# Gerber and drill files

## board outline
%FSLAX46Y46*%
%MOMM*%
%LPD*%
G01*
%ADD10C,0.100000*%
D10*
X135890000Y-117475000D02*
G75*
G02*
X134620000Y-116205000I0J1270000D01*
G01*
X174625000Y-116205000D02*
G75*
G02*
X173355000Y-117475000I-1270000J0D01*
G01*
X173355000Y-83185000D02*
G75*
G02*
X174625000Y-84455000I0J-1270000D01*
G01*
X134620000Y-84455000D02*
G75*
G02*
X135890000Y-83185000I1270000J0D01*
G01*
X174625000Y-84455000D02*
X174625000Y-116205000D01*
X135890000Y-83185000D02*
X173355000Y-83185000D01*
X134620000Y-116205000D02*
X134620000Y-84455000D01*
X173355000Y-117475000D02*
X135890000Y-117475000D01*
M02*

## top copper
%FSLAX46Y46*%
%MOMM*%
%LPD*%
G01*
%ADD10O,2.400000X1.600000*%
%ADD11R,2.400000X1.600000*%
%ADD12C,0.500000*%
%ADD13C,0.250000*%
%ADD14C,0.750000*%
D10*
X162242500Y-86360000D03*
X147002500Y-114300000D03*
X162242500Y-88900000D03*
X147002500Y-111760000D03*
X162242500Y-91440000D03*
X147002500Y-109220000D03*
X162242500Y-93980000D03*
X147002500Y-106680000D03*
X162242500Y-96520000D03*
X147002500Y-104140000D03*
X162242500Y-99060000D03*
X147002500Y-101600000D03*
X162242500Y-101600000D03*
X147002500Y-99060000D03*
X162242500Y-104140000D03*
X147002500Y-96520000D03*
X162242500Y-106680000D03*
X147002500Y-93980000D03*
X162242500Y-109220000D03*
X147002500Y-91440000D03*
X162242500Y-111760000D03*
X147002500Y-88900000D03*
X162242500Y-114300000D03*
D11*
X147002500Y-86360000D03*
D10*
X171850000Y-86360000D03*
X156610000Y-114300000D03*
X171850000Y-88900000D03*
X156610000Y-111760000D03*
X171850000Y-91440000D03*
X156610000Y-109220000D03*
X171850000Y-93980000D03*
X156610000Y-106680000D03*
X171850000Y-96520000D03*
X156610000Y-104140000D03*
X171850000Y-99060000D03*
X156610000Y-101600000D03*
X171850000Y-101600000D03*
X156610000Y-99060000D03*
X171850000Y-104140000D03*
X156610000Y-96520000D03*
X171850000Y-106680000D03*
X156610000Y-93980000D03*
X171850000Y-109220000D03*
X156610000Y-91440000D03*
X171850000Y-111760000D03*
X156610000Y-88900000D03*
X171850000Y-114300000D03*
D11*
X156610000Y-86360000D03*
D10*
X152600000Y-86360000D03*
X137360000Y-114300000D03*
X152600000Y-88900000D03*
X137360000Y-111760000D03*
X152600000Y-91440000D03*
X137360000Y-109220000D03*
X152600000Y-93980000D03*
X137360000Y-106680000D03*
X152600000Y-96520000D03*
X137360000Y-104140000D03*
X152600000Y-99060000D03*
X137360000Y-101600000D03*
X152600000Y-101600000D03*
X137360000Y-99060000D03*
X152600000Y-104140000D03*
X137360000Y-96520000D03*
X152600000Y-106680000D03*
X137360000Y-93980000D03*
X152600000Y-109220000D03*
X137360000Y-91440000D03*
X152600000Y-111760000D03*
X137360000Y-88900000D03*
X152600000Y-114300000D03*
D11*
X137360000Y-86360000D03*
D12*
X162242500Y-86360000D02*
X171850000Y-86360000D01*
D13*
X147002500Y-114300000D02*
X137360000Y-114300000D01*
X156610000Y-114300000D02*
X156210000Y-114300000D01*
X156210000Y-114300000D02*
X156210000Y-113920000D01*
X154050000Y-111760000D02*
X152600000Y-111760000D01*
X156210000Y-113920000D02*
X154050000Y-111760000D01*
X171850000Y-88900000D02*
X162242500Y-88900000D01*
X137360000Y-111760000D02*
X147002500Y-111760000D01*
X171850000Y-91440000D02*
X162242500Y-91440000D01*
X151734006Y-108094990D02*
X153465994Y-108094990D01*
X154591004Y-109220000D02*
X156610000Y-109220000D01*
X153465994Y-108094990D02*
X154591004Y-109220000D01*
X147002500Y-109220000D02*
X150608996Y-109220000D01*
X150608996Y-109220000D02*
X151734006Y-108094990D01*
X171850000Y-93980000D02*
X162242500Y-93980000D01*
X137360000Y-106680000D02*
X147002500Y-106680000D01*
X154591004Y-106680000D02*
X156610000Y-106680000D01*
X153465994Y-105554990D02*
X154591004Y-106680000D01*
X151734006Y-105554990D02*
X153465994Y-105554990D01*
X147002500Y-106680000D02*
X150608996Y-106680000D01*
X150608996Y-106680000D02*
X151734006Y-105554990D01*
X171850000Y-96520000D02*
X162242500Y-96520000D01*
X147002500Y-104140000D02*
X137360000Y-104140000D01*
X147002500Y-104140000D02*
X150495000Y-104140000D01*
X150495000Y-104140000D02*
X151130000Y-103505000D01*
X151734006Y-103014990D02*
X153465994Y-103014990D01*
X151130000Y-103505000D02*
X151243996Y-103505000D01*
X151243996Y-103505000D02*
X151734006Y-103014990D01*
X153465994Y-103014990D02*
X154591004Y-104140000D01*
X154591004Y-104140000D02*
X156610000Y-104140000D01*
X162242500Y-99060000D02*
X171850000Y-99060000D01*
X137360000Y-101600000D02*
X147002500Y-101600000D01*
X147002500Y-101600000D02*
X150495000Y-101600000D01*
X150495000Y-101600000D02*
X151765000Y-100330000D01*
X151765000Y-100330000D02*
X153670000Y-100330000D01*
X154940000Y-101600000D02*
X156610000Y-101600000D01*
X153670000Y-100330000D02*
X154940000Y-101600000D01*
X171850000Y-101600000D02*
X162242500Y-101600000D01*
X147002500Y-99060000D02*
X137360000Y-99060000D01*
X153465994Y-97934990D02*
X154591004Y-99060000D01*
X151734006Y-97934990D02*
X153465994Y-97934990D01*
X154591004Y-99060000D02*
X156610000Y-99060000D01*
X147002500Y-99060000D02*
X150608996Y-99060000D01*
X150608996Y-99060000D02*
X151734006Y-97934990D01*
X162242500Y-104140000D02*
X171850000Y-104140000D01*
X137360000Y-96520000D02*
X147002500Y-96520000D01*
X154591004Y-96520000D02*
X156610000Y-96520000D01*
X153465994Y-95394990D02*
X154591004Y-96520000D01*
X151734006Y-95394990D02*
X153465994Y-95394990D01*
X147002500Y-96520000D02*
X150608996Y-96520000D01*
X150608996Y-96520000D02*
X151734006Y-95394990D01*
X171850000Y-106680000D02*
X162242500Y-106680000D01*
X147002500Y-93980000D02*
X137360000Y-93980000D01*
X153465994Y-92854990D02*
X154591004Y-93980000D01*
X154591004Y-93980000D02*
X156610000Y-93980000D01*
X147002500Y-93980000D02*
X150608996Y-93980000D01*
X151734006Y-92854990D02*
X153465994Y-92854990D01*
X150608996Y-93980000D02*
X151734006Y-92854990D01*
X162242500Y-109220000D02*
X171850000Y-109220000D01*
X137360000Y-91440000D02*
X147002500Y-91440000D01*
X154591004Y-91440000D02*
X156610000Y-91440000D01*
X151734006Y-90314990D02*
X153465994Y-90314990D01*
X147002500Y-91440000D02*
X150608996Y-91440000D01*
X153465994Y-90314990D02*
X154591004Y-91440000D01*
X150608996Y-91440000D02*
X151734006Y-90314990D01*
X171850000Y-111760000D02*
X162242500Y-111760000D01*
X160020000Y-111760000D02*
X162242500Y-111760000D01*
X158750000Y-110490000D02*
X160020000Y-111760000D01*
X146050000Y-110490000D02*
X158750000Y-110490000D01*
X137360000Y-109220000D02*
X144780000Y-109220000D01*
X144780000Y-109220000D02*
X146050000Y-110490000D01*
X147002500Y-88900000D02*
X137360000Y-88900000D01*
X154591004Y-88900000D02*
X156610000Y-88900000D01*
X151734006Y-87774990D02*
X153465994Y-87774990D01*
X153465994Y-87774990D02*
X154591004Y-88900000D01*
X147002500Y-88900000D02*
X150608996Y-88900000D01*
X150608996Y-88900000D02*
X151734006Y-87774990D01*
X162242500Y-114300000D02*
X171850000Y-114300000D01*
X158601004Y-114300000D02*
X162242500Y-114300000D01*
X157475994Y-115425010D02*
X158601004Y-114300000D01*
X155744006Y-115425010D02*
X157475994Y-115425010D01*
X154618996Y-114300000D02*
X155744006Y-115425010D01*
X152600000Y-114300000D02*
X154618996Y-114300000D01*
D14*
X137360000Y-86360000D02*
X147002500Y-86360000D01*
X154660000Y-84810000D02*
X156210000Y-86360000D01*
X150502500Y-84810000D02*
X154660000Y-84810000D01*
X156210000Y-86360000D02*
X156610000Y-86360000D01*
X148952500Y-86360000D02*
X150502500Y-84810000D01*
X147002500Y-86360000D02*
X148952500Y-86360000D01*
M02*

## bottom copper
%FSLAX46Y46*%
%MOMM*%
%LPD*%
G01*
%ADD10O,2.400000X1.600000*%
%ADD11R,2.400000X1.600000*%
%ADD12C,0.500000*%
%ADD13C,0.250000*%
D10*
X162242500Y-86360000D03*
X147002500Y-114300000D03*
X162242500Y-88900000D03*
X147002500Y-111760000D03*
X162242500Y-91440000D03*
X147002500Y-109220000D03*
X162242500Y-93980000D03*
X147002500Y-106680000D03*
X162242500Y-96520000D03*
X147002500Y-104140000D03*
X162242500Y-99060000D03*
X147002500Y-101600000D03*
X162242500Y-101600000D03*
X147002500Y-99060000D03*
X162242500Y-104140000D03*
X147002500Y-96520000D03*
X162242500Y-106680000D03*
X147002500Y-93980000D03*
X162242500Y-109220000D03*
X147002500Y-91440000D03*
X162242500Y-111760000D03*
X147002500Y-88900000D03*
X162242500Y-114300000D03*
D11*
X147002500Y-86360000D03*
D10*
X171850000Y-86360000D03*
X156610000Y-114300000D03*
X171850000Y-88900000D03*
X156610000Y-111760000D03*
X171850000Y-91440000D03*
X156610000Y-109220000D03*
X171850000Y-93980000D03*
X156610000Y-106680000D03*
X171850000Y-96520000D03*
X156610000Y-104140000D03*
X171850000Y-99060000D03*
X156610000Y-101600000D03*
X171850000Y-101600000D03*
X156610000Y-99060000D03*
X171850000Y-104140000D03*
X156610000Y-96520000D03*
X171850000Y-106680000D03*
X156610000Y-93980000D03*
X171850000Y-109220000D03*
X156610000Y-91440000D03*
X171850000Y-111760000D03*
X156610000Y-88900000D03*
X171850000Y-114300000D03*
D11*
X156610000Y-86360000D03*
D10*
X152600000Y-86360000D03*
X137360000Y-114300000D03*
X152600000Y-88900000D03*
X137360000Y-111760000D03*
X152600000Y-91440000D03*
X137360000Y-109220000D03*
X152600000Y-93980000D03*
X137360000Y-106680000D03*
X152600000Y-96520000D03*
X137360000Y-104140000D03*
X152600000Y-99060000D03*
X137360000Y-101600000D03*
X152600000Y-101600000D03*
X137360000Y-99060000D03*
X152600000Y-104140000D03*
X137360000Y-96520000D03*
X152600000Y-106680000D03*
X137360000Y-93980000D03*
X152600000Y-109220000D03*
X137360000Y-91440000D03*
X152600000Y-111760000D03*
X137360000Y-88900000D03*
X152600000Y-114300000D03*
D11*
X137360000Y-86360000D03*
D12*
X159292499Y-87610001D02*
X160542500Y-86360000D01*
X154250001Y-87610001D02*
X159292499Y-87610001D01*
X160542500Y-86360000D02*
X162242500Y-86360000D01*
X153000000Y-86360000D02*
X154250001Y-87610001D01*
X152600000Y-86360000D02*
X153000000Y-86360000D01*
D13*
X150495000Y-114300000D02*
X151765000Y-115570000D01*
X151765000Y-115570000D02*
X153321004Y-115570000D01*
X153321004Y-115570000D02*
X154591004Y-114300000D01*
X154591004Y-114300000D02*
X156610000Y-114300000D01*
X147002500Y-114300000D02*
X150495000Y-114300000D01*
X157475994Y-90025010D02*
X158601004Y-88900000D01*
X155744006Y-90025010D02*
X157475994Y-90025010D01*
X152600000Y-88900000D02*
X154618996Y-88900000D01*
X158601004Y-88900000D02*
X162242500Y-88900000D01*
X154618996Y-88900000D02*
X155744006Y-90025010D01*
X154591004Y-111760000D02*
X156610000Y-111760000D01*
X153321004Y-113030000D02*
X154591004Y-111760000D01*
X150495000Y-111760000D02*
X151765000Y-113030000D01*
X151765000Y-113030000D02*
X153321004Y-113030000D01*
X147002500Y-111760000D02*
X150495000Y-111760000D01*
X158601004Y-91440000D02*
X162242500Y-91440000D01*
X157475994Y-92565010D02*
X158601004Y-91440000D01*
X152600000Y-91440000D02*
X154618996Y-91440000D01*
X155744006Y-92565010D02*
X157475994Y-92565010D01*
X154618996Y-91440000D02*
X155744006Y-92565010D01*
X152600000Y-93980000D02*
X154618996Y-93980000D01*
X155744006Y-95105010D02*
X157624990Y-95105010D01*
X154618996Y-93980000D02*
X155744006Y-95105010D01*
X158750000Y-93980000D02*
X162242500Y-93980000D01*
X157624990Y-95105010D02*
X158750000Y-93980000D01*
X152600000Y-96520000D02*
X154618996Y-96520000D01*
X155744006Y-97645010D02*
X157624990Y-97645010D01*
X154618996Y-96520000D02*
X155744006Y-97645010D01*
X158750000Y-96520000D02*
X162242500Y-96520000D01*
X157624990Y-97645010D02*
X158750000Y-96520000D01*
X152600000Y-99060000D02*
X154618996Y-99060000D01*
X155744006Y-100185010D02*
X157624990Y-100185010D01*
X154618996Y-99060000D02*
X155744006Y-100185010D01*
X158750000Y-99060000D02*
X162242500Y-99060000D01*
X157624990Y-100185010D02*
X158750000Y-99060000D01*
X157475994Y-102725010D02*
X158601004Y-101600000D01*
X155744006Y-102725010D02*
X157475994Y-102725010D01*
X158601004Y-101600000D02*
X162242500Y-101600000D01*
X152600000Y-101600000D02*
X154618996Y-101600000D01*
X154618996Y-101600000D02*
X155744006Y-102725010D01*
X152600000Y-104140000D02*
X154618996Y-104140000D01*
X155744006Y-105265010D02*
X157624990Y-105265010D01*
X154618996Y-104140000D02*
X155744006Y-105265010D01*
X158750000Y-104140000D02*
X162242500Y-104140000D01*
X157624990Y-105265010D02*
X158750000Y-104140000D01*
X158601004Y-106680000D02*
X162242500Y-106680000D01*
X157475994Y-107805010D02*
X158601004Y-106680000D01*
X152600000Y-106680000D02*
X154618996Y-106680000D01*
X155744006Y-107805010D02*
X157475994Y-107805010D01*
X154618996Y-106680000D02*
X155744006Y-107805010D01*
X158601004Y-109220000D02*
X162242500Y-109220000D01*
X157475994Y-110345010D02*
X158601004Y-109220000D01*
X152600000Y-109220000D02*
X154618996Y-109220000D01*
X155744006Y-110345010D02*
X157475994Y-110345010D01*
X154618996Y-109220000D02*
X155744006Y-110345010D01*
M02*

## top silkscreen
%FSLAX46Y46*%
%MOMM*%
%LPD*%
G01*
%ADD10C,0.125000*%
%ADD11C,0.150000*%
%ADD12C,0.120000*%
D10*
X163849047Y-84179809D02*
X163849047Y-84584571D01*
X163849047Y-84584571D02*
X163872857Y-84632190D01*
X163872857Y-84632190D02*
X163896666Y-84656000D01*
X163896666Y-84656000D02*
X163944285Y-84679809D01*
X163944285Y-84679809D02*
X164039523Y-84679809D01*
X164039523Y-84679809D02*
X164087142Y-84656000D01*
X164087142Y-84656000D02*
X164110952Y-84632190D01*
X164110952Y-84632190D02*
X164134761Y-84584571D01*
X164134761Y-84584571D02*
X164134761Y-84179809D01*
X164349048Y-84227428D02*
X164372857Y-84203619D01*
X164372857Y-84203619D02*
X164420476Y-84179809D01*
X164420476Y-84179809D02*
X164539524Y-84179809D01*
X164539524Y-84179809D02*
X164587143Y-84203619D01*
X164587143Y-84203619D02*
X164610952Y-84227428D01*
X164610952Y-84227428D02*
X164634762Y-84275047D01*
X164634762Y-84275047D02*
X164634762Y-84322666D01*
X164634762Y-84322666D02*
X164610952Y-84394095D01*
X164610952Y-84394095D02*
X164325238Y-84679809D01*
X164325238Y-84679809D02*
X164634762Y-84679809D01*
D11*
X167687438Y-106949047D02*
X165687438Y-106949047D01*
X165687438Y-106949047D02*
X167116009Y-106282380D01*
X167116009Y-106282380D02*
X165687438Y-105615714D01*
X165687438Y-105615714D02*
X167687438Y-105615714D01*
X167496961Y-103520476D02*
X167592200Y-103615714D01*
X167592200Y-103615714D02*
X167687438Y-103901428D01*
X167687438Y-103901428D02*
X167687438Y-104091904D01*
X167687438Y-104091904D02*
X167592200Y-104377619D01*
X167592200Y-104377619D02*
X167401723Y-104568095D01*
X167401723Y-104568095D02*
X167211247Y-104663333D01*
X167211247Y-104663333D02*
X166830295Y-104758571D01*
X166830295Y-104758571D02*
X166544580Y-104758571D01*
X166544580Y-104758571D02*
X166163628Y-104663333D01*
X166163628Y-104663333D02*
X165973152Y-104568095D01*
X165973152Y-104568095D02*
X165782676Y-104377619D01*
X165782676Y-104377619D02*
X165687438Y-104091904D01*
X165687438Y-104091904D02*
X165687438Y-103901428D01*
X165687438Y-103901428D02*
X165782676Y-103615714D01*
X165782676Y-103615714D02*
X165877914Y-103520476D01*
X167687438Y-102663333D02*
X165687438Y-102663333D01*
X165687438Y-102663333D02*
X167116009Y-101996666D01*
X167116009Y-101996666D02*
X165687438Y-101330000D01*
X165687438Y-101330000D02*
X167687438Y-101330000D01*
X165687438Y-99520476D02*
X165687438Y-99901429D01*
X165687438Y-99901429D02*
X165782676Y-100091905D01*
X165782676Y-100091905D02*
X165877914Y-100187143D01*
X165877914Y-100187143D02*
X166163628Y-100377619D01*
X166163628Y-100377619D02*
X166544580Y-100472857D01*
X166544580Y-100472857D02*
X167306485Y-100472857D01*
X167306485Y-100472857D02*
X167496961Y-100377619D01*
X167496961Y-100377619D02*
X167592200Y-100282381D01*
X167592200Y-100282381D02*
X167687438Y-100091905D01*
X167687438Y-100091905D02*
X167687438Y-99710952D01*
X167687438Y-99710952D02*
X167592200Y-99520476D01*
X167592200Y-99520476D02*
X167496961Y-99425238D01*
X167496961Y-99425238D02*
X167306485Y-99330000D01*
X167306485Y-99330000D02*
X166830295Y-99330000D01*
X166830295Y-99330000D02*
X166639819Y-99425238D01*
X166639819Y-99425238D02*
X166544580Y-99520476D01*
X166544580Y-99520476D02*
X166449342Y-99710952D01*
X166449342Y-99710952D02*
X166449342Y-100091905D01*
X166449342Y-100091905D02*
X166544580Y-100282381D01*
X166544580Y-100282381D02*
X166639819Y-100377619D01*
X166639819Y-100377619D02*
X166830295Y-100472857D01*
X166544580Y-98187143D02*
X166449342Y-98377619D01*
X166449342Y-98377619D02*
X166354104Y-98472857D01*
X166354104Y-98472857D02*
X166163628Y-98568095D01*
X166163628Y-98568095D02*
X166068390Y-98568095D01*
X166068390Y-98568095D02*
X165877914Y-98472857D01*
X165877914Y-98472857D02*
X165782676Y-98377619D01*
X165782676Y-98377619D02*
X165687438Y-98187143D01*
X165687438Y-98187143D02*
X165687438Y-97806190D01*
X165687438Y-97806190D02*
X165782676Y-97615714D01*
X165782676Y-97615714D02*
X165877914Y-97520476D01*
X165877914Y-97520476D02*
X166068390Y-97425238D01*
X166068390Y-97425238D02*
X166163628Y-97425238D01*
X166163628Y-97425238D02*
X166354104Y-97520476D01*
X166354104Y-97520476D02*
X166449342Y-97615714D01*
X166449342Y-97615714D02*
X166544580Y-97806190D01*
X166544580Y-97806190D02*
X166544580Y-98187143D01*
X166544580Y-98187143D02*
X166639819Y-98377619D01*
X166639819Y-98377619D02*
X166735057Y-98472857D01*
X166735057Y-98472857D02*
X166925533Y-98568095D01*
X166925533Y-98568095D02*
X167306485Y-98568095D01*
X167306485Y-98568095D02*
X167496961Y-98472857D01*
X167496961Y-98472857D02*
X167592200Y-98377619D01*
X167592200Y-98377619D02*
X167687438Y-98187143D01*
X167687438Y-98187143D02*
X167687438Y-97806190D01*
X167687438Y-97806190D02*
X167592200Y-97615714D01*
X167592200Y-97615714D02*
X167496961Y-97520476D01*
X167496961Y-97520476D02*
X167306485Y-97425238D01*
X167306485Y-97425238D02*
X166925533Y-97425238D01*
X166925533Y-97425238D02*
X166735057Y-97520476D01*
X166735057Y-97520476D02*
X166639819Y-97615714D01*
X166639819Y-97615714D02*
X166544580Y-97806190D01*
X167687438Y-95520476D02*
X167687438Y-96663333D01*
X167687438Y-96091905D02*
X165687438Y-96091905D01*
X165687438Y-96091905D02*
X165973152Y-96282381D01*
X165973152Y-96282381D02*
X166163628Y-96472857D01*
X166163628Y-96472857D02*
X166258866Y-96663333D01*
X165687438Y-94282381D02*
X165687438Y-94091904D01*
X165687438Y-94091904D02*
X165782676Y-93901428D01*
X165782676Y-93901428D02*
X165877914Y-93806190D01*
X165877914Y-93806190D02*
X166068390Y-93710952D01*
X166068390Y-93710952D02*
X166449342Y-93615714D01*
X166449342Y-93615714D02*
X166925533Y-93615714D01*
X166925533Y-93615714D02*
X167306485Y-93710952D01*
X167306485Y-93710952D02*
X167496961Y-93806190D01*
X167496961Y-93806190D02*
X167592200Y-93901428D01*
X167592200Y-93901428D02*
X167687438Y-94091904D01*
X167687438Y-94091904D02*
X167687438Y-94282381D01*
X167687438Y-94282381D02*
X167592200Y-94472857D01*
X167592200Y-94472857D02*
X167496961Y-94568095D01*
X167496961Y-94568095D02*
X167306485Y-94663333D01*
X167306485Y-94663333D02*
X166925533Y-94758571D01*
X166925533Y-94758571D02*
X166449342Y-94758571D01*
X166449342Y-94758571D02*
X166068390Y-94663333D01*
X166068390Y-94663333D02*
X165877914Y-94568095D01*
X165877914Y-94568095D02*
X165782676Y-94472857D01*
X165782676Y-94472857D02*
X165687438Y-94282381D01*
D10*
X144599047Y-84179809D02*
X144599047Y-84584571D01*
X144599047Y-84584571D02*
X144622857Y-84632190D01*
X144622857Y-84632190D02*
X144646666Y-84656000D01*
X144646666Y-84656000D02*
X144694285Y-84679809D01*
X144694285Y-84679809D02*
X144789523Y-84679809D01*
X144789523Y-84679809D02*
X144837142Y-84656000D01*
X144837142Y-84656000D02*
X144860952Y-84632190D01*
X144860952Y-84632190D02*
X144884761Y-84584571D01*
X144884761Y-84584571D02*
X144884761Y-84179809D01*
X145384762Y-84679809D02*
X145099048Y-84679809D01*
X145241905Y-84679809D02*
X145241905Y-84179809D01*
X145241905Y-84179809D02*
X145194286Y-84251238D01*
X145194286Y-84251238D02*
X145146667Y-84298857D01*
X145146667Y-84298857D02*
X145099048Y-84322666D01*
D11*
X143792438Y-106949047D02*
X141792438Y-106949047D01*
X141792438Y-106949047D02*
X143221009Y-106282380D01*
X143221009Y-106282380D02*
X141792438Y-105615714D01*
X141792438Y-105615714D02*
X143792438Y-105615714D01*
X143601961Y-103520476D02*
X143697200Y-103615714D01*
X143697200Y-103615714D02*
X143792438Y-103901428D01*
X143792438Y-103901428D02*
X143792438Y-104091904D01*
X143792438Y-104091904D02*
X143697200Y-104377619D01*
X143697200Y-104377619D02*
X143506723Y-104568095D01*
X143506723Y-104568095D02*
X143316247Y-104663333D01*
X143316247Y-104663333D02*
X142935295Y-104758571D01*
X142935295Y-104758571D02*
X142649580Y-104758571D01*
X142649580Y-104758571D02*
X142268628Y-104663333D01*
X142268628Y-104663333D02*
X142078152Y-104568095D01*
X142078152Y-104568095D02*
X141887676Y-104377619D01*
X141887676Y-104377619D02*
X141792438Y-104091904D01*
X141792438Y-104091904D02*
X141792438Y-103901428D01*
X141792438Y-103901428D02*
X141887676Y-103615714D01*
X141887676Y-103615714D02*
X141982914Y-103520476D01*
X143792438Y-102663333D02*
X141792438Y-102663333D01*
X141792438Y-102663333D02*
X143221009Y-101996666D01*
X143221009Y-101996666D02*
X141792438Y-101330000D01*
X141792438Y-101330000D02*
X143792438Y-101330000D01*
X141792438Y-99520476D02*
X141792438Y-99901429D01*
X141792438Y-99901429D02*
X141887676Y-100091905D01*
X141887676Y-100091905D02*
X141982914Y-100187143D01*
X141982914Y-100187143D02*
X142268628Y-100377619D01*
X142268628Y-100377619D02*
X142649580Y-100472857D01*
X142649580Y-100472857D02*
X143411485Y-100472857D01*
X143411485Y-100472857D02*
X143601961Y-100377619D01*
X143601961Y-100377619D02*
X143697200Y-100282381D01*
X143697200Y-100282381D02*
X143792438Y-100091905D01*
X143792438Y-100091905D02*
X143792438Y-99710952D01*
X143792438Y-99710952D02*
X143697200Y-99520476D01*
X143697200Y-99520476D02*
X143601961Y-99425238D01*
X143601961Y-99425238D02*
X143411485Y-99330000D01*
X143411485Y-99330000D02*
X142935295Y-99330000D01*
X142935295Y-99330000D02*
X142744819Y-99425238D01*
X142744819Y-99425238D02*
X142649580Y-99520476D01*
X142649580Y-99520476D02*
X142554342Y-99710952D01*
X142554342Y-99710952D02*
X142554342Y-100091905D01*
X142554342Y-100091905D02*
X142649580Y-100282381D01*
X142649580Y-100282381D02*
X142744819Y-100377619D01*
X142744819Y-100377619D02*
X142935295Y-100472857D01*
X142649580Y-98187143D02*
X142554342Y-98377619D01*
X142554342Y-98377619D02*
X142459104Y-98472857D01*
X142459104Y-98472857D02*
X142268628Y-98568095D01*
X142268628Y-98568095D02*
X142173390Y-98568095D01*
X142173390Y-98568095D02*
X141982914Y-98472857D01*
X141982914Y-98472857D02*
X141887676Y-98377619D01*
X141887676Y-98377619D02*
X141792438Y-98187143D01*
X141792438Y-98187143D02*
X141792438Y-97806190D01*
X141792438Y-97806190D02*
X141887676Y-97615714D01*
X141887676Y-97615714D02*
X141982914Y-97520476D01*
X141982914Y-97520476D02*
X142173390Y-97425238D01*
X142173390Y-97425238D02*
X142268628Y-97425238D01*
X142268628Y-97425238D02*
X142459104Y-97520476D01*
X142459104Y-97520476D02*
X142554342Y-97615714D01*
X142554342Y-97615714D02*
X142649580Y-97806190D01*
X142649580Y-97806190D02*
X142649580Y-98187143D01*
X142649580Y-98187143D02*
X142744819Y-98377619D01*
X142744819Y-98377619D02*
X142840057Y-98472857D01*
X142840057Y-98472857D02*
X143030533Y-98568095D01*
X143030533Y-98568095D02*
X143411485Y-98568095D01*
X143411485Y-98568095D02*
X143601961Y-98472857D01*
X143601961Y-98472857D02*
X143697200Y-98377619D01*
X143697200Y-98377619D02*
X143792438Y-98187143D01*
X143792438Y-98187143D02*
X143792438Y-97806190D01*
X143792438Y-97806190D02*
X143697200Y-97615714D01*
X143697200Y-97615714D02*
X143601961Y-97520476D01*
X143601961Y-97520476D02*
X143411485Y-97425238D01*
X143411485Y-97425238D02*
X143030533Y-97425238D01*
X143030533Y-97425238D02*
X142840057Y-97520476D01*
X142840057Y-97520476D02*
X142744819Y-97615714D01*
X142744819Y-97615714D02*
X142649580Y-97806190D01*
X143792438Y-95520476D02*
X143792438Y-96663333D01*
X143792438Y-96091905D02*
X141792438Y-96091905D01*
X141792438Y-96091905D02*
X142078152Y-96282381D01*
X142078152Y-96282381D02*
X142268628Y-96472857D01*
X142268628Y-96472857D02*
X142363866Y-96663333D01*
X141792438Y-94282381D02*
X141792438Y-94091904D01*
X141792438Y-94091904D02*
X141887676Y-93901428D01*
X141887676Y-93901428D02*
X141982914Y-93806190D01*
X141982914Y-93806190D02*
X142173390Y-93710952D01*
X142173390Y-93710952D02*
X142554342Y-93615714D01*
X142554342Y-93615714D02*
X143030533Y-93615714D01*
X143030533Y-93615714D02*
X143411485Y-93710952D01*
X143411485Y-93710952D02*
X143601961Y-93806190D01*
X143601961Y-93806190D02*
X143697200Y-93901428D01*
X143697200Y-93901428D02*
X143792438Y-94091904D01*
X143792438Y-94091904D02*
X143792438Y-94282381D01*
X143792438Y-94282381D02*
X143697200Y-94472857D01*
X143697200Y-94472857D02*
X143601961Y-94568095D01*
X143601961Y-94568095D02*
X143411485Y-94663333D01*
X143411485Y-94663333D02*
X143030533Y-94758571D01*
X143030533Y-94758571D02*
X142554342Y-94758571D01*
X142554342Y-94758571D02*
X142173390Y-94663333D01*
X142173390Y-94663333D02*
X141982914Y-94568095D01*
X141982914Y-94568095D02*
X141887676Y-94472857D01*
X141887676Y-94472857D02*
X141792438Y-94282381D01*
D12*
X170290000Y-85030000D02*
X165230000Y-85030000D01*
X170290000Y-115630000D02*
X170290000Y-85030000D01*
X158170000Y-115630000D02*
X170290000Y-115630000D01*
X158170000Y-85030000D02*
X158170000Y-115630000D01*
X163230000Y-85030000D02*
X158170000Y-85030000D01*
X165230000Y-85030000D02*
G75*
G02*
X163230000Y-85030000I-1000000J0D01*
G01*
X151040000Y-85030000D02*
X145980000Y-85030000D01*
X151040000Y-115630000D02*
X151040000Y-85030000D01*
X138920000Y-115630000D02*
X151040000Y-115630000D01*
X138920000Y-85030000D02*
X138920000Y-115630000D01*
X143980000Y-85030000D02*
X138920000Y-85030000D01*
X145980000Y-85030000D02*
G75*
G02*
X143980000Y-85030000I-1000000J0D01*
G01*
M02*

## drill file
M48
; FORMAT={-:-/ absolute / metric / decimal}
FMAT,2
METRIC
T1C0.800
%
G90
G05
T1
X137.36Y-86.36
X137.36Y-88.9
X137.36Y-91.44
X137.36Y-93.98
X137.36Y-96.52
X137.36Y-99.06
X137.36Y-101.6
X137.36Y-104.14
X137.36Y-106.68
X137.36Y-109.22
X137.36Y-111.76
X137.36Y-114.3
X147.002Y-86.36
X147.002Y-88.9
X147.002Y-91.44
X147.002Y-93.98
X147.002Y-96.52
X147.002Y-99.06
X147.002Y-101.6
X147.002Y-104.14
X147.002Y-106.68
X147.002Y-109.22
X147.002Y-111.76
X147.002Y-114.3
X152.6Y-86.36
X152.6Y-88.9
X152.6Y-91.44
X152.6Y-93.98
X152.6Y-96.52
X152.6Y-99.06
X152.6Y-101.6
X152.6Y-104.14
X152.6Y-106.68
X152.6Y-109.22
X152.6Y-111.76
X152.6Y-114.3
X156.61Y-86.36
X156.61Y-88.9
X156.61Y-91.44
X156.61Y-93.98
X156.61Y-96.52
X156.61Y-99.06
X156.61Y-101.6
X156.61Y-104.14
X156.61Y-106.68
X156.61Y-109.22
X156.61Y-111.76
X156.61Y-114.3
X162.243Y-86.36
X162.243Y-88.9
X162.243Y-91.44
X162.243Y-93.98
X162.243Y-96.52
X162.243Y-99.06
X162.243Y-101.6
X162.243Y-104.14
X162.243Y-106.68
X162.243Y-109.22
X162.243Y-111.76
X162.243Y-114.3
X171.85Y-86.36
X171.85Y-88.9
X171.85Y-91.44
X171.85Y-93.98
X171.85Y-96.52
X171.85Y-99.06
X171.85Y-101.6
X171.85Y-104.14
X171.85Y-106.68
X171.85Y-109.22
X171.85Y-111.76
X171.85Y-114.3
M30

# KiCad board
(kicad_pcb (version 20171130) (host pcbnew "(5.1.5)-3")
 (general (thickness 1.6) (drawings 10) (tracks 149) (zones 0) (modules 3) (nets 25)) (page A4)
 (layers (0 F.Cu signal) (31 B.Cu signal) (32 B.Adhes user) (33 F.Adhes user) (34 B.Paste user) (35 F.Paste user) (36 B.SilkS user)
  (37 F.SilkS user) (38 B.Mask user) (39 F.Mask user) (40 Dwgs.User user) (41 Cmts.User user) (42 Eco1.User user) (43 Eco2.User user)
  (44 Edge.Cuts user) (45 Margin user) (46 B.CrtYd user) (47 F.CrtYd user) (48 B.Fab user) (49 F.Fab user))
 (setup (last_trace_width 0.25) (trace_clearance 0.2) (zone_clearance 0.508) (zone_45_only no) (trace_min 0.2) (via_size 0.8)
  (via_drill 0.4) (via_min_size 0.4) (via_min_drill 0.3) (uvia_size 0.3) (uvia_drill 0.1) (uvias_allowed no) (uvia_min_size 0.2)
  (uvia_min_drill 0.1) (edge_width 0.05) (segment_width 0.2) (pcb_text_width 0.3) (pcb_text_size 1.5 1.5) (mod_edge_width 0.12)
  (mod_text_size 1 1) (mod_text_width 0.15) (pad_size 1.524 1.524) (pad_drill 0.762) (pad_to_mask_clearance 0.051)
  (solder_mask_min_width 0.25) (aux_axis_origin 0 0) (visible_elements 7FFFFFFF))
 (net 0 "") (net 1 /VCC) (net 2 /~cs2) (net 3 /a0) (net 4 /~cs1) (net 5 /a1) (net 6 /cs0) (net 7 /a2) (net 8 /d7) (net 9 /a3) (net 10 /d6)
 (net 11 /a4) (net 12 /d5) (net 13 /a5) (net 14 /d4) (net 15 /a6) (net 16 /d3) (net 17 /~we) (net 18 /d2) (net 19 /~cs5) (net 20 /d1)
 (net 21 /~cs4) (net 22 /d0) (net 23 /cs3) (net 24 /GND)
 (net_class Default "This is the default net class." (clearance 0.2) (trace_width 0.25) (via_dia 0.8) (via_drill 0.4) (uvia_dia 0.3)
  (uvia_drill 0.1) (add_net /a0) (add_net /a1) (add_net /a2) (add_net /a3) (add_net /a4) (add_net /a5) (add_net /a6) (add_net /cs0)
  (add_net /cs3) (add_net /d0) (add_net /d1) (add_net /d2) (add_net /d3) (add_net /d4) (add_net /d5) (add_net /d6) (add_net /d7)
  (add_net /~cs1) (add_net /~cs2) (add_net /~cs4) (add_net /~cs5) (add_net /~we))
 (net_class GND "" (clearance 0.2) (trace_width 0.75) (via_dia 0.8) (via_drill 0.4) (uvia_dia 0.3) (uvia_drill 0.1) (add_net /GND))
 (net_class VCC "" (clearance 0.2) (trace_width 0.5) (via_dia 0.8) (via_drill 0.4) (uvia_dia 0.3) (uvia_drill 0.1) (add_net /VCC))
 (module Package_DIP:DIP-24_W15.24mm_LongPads (layer F.Cu) (at 147.0025 86.36)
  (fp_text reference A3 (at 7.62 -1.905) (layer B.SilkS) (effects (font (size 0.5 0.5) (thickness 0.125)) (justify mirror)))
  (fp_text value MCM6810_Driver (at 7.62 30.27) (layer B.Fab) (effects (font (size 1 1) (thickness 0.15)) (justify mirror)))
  (pad 24 thru_hole oval (at 15.24 0) (size 2.4 1.6) (drill 0.8) (layers *.Cu *.Mask) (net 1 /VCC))
  (pad 12 thru_hole oval (at 0 27.94) (size 2.4 1.6) (drill 0.8) (layers *.Cu *.Mask) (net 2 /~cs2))
  (pad 23 thru_hole oval (at 15.24 2.54) (size 2.4 1.6) (drill 0.8) (layers *.Cu *.Mask) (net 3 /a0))
  (pad 11 thru_hole oval (at 0 25.4) (size 2.4 1.6) (drill 0.8) (layers *.Cu *.Mask) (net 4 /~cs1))
  (pad 22 thru_hole oval (at 15.24 5.08) (size 2.4 1.6) (drill 0.8) (layers *.Cu *.Mask) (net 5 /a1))
  (pad 10 thru_hole oval (at 0 22.86) (size 2.4 1.6) (drill 0.8) (layers *.Cu *.Mask) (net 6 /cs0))
  (pad 21 thru_hole oval (at 15.24 7.62) (size 2.4 1.6) (drill 0.8) (layers *.Cu *.Mask) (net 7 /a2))
  (pad 9 thru_hole oval (at 0 20.32) (size 2.4 1.6) (drill 0.8) (layers *.Cu *.Mask) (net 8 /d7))
  (pad 20 thru_hole oval (at 15.24 10.16) (size 2.4 1.6) (drill 0.8) (layers *.Cu *.Mask) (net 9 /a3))
  (pad 8 thru_hole oval (at 0 17.78) (size 2.4 1.6) (drill 0.8) (layers *.Cu *.Mask) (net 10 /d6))
  (pad 19 thru_hole oval (at 15.24 12.7) (size 2.4 1.6) (drill 0.8) (layers *.Cu *.Mask) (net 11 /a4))
  (pad 7 thru_hole oval (at 0 15.24) (size 2.4 1.6) (drill 0.8) (layers *.Cu *.Mask) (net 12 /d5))
  (pad 18 thru_hole oval (at 15.24 15.24) (size 2.4 1.6) (drill 0.8) (layers *.Cu *.Mask) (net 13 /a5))
  (pad 6 thru_hole oval (at 0 12.7) (size 2.4 1.6) (drill 0.8) (layers *.Cu *.Mask) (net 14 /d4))
  (pad 17 thru_hole oval (at 15.24 17.78) (size 2.4 1.6) (drill 0.8) (layers *.Cu *.Mask) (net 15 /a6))
  (pad 5 thru_hole oval (at 0 10.16) (size 2.4 1.6) (drill 0.8) (layers *.Cu *.Mask) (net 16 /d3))
  (pad 16 thru_hole oval (at 15.24 20.32) (size 2.4 1.6) (drill 0.8) (layers *.Cu *.Mask) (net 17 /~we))
  (pad 4 thru_hole oval (at 0 7.62) (size 2.4 1.6) (drill 0.8) (layers *.Cu *.Mask) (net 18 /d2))
  (pad 15 thru_hole oval (at 15.24 22.86) (size 2.4 1.6) (drill 0.8) (layers *.Cu *.Mask) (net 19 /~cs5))
  (pad 3 thru_hole oval (at 0 5.08) (size 2.4 1.6) (drill 0.8) (layers *.Cu *.Mask) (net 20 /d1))
  (pad 14 thru_hole oval (at 15.24 25.4) (size 2.4 1.6) (drill 0.8) (layers *.Cu *.Mask) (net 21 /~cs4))
  (pad 2 thru_hole oval (at 0 2.54) (size 2.4 1.6) (drill 0.8) (layers *.Cu *.Mask) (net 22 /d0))
  (pad 13 thru_hole oval (at 15.24 27.94) (size 2.4 1.6) (drill 0.8) (layers *.Cu *.Mask) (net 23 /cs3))
  (pad 1 thru_hole rect (at 0 0) (size 2.4 1.6) (drill 0.8) (layers *.Cu *.Mask) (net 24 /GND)))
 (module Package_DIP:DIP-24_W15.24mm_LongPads (layer F.Cu) (at 156.61 86.36)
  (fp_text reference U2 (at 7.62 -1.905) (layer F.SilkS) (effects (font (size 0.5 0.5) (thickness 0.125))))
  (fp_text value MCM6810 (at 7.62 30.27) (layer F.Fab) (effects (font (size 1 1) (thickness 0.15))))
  (fp_line (start 13.68 -1.33) (end 8.62 -1.33) (layer F.SilkS) (width 0.12))
  (fp_line (start 13.68 29.27) (end 13.68 -1.33) (layer F.SilkS) (width 0.12))
  (fp_line (start 1.56 29.27) (end 13.68 29.27) (layer F.SilkS) (width 0.12))
  (fp_line (start 1.56 -1.33) (end 1.56 29.27) (layer F.SilkS) (width 0.12))
  (fp_line (start 6.62 -1.33) (end 1.56 -1.33) (layer F.SilkS) (width 0.12))
  (fp_arc (start 7.62 -1.33) (end 6.62 -1.33) (angle -180) (layer F.SilkS) (width 0.12))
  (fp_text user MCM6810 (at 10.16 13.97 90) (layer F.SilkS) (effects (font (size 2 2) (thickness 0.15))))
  (pad 24 thru_hole oval (at 15.24 0) (size 2.4 1.6) (drill 0.8) (layers *.Cu *.Mask) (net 1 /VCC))
  (pad 12 thru_hole oval (at 0 27.94) (size 2.4 1.6) (drill 0.8) (layers *.Cu *.Mask) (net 2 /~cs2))
  (pad 23 thru_hole oval (at 15.24 2.54) (size 2.4 1.6) (drill 0.8) (layers *.Cu *.Mask) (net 3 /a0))
  (pad 11 thru_hole oval (at 0 25.4) (size 2.4 1.6) (drill 0.8) (layers *.Cu *.Mask) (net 4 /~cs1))
  (pad 22 thru_hole oval (at 15.24 5.08) (size 2.4 1.6) (drill 0.8) (layers *.Cu *.Mask) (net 5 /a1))
  (pad 10 thru_hole oval (at 0 22.86) (size 2.4 1.6) (drill 0.8) (layers *.Cu *.Mask) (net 6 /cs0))
  (pad 21 thru_hole oval (at 15.24 7.62) (size 2.4 1.6) (drill 0.8) (layers *.Cu *.Mask) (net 7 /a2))
  (pad 9 thru_hole oval (at 0 20.32) (size 2.4 1.6) (drill 0.8) (layers *.Cu *.Mask) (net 8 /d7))
  (pad 20 thru_hole oval (at 15.24 10.16) (size 2.4 1.6) (drill 0.8) (layers *.Cu *.Mask) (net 9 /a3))
  (pad 8 thru_hole oval (at 0 17.78) (size 2.4 1.6) (drill 0.8) (layers *.Cu *.Mask) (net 10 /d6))
  (pad 19 thru_hole oval (at 15.24 12.7) (size 2.4 1.6) (drill 0.8) (layers *.Cu *.Mask) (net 11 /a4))
  (pad 7 thru_hole oval (at 0 15.24) (size 2.4 1.6) (drill 0.8) (layers *.Cu *.Mask) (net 12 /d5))
  (pad 18 thru_hole oval (at 15.24 15.24) (size 2.4 1.6) (drill 0.8) (layers *.Cu *.Mask) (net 13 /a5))
  (pad 6 thru_hole oval (at 0 12.7) (size 2.4 1.6) (drill 0.8) (layers *.Cu *.Mask) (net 14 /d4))
  (pad 17 thru_hole oval (at 15.24 17.78) (size 2.4 1.6) (drill 0.8) (layers *.Cu *.Mask) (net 15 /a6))
  (pad 5 thru_hole oval (at 0 10.16) (size 2.4 1.6) (drill 0.8) (layers *.Cu *.Mask) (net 16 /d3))
  (pad 16 thru_hole oval (at 15.24 20.32) (size 2.4 1.6) (drill 0.8) (layers *.Cu *.Mask) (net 17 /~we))
  (pad 4 thru_hole oval (at 0 7.62) (size 2.4 1.6) (drill 0.8) (layers *.Cu *.Mask) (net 18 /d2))
  (pad 15 thru_hole oval (at 15.24 22.86) (size 2.4 1.6) (drill 0.8) (layers *.Cu *.Mask) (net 19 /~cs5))
  (pad 3 thru_hole oval (at 0 5.08) (size 2.4 1.6) (drill 0.8) (layers *.Cu *.Mask) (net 20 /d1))
  (pad 14 thru_hole oval (at 15.24 25.4) (size 2.4 1.6) (drill 0.8) (layers *.Cu *.Mask) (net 21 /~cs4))
  (pad 2 thru_hole oval (at 0 2.54) (size 2.4 1.6) (drill 0.8) (layers *.Cu *.Mask) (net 22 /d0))
  (pad 13 thru_hole oval (at 15.24 27.94) (size 2.4 1.6) (drill 0.8) (layers *.Cu *.Mask) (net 23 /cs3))
  (pad 1 thru_hole rect (at 0 0) (size 2.4 1.6) (drill 0.8) (layers *.Cu *.Mask) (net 24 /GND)))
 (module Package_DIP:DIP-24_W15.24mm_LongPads (layer F.Cu) (at 137.36 86.36)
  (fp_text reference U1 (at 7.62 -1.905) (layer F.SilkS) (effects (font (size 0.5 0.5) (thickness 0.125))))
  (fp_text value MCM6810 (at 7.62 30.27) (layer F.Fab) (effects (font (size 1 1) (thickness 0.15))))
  (fp_line (start 13.68 -1.33) (end 8.62 -1.33) (layer F.SilkS) (width 0.12))
  (fp_line (start 13.68 29.27) (end 13.68 -1.33) (layer F.SilkS) (width 0.12))
  (fp_line (start 1.56 29.27) (end 13.68 29.27) (layer F.SilkS) (width 0.12))
  (fp_line (start 1.56 -1.33) (end 1.56 29.27) (layer F.SilkS) (width 0.12))
  (fp_line (start 6.62 -1.33) (end 1.56 -1.33) (layer F.SilkS) (width 0.12))
  (fp_arc (start 7.62 -1.33) (end 6.62 -1.33) (angle -180) (layer F.SilkS) (width 0.12))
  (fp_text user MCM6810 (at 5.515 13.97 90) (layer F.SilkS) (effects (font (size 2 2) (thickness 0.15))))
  (pad 24 thru_hole oval (at 15.24 0) (size 2.4 1.6) (drill 0.8) (layers *.Cu *.Mask) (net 1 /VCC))
  (pad 12 thru_hole oval (at 0 27.94) (size 2.4 1.6) (drill 0.8) (layers *.Cu *.Mask) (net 2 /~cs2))
  (pad 23 thru_hole oval (at 15.24 2.54) (size 2.4 1.6) (drill 0.8) (layers *.Cu *.Mask) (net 3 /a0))
  (pad 11 thru_hole oval (at 0 25.4) (size 2.4 1.6) (drill 0.8) (layers *.Cu *.Mask) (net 4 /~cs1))
  (pad 22 thru_hole oval (at 15.24 5.08) (size 2.4 1.6) (drill 0.8) (layers *.Cu *.Mask) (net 5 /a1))
  (pad 10 thru_hole oval (at 0 22.86) (size 2.4 1.6) (drill 0.8) (layers *.Cu *.Mask) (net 21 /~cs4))
  (pad 21 thru_hole oval (at 15.24 7.62) (size 2.4 1.6) (drill 0.8) (layers *.Cu *.Mask) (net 7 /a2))
  (pad 9 thru_hole oval (at 0 20.32) (size 2.4 1.6) (drill 0.8) (layers *.Cu *.Mask) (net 8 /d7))
  (pad 20 thru_hole oval (at 15.24 10.16) (size 2.4 1.6) (drill 0.8) (layers *.Cu *.Mask) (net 9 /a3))
  (pad 8 thru_hole oval (at 0 17.78) (size 2.4 1.6) (drill 0.8) (layers *.Cu *.Mask) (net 10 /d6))
  (pad 19 thru_hole oval (at 15.24 12.7) (size 2.4 1.6) (drill 0.8) (layers *.Cu *.Mask) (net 11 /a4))
  (pad 7 thru_hole oval (at 0 15.24) (size 2.4 1.6) (drill 0.8) (layers *.Cu *.Mask) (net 12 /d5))
  (pad 18 thru_hole oval (at 15.24 15.24) (size 2.4 1.6) (drill 0.8) (layers *.Cu *.Mask) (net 13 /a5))
  (pad 6 thru_hole oval (at 0 12.7) (size 2.4 1.6) (drill 0.8) (layers *.Cu *.Mask) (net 14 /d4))
  (pad 17 thru_hole oval (at 15.24 17.78) (size 2.4 1.6) (drill 0.8) (layers *.Cu *.Mask) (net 15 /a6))
  (pad 5 thru_hole oval (at 0 10.16) (size 2.4 1.6) (drill 0.8) (layers *.Cu *.Mask) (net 16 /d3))
  (pad 16 thru_hole oval (at 15.24 20.32) (size 2.4 1.6) (drill 0.8) (layers *.Cu *.Mask) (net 17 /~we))
  (pad 4 thru_hole oval (at 0 7.62) (size 2.4 1.6) (drill 0.8) (layers *.Cu *.Mask) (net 18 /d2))
  (pad 15 thru_hole oval (at 15.24 22.86) (size 2.4 1.6) (drill 0.8) (layers *.Cu *.Mask) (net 19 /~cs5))
  (pad 3 thru_hole oval (at 0 5.08) (size 2.4 1.6) (drill 0.8) (layers *.Cu *.Mask) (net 20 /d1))
  (pad 14 thru_hole oval (at 15.24 25.4) (size 2.4 1.6) (drill 0.8) (layers *.Cu *.Mask) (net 2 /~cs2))
  (pad 2 thru_hole oval (at 0 2.54) (size 2.4 1.6) (drill 0.8) (layers *.Cu *.Mask) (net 22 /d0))
  (pad 13 thru_hole oval (at 15.24 27.94) (size 2.4 1.6) (drill 0.8) (layers *.Cu *.Mask) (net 23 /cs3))
  (pad 1 thru_hole rect (at 0 0) (size 2.4 1.6) (drill 0.8) (layers *.Cu *.Mask) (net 24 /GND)))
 (gr_arc (start 135.89 116.205) (end 134.62 116.205) (angle -90) (layer Edge.Cuts) (width 0.1))
 (gr_arc (start 173.355 116.205) (end 173.355 117.475) (angle -90) (layer Edge.Cuts) (width 0.1))
 (gr_arc (start 173.355 84.455) (end 174.625 84.455) (angle -90) (layer Edge.Cuts) (width 0.1))
 (gr_arc (start 135.89 84.455) (end 135.89 83.185) (angle -90) (layer Edge.Cuts) (width 0.1))
 (gr_line (start 174.625 84.455) (end 174.625 116.205) (layer Edge.Cuts) (width 0.1))
 (gr_line (start 135.89 83.185) (end 173.355 83.185) (layer Edge.Cuts) (width 0.1))
 (gr_line (start 134.62 116.205) (end 134.62 84.455) (layer Edge.Cuts) (width 0.1))
 (gr_line (start 173.355 117.475) (end 135.89 117.475) (layer Edge.Cuts) (width 0.1))
 (segment (start 159.292499 87.610001) (end 160.5425 86.36) (width 0.5) (layer B.Cu) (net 1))
 (segment (start 154.250001 87.610001) (end 159.292499 87.610001) (width 0.5) (layer B.Cu) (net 1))
 (segment (start 160.5425 86.36) (end 162.2425 86.36) (width 0.5) (layer B.Cu) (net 1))
 (segment (start 153 86.36) (end 154.250001 87.610001) (width 0.5) (layer B.Cu) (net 1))
 (segment (start 152.6 86.36) (end 153 86.36) (width 0.5) (layer B.Cu) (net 1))
 (segment (start 162.2425 86.36) (end 171.85 86.36) (width 0.5) (layer F.Cu) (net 1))
 (segment (start 147.0025 114.3) (end 137.36 114.3) (width 0.25) (layer F.Cu) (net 2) (status 30))
 (segment (start 156.61 114.3) (end 156.21 114.3) (width 0.25) (layer F.Cu) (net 2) (status 30))
 (segment (start 156.21 114.3) (end 156.21 113.92) (width 0.25) (layer F.Cu) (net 2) (status 30))
 (segment (start 150.495 114.3) (end 151.765 115.57) (width 0.25) (layer B.Cu) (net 2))
 (segment (start 151.765 115.57) (end 153.321004 115.57) (width 0.25) (layer B.Cu) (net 2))
 (segment (start 153.321004 115.57) (end 154.591004 114.3) (width 0.25) (layer B.Cu) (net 2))
 (segment (start 154.591004 114.3) (end 156.61 114.3) (width 0.25) (layer B.Cu) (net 2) (status 20))
 (segment (start 147.0025 114.3) (end 150.495 114.3) (width 0.25) (layer B.Cu) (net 2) (status 10))
 (segment (start 154.05 111.76) (end 152.6 111.76) (width 0.25) (layer F.Cu) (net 2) (status 20))
 (segment (start 156.21 113.92) (end 154.05 111.76) (width 0.25) (layer F.Cu) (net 2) (status 10))
 (segment (start 171.85 88.9) (end 162.2425 88.9) (width 0.25) (layer F.Cu) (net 3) (status 30))
 (segment (start 157.475994 90.02501) (end 158.601004 88.9) (width 0.25) (layer B.Cu) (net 3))
 (segment (start 155.744006 90.02501) (end 157.475994 90.02501) (width 0.25) (layer B.Cu) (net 3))
 (segment (start 152.6 88.9) (end 154.618996 88.9) (width 0.25) (layer B.Cu) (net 3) (status 10))
 (segment (start 158.601004 88.9) (end 162.2425 88.9) (width 0.25) (layer B.Cu) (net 3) (status 20))
 (segment (start 154.618996 88.9) (end 155.744006 90.02501) (width 0.25) (layer B.Cu) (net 3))
 (segment (start 137.36 111.76) (end 147.0025 111.76) (width 0.25) (layer F.Cu) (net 4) (status 30))
 (segment (start 154.591004 111.76) (end 156.61 111.76) (width 0.25) (layer B.Cu) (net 4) (status 20))
 (segment (start 153.321004 113.03) (end 154.591004 111.76) (width 0.25) (layer B.Cu) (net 4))
 (segment (start 150.495 111.76) (end 151.765 113.03) (width 0.25) (layer B.Cu) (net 4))
 (segment (start 151.765 113.03) (end 153.321004 113.03) (width 0.25) (layer B.Cu) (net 4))
 (segment (start 147.0025 111.76) (end 150.495 111.76) (width 0.25) (layer B.Cu) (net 4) (status 10))
 (segment (start 171.85 91.44) (end 162.2425 91.44) (width 0.25) (layer F.Cu) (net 5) (status 30))
 (segment (start 158.601004 91.44) (end 162.2425 91.44) (width 0.25) (layer B.Cu) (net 5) (status 20))
 (segment (start 157.475994 92.56501) (end 158.601004 91.44) (width 0.25) (layer B.Cu) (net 5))
 (segment (start 152.6 91.44) (end 154.618996 91.44) (width 0.25) (layer B.Cu) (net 5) (status 10))
 (segment (start 155.744006 92.56501) (end 157.475994 92.56501) (width 0.25) (layer B.Cu) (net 5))
 (segment (start 154.618996 91.44) (end 155.744006 92.56501) (width 0.25) (layer B.Cu) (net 5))
 (segment (start 151.734006 108.09499) (end 153.465994 108.09499) (width 0.25) (layer F.Cu) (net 6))
 (segment (start 154.591004 109.22) (end 156.61 109.22) (width 0.25) (layer F.Cu) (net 6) (status 20))
 (segment (start 153.465994 108.09499) (end 154.591004 109.22) (width 0.25) (layer F.Cu) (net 6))
 (segment (start 147.0025 109.22) (end 150.608996 109.22) (width 0.25) (layer F.Cu) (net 6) (status 10))
 (segment (start 150.608996 109.22) (end 151.734006 108.09499) (width 0.25) (layer F.Cu) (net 6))
 (segment (start 171.85 93.98) (end 162.2425 93.98) (width 0.25) (layer F.Cu) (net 7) (status 30))
 (segment (start 152.6 93.98) (end 154.618996 93.98) (width 0.25) (layer B.Cu) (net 7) (status 10))
 (segment (start 155.744006 95.10501) (end 157.62499 95.10501) (width 0.25) (layer B.Cu) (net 7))
 (segment (start 154.618996 93.98) (end 155.744006 95.10501) (width 0.25) (layer B.Cu) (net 7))
 (segment (start 158.75 93.98) (end 162.2425 93.98) (width 0.25) (layer B.Cu) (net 7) (status 20))
 (segment (start 157.62499 95.10501) (end 158.75 93.98) (width 0.25) (layer B.Cu) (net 7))
 (segment (start 137.36 106.68) (end 147.0025 106.68) (width 0.25) (layer F.Cu) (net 8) (status 30))
 (segment (start 154.591004 106.68) (end 156.61 106.68) (width 0.25) (layer F.Cu) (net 8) (status 20))
 (segment (start 153.465994 105.55499) (end 154.591004 106.68) (width 0.25) (layer F.Cu) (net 8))
 (segment (start 151.734006 105.55499) (end 153.465994 105.55499) (width 0.25) (layer F.Cu) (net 8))
 (segment (start 147.0025 106.68) (end 150.608996 106.68) (width 0.25) (layer F.Cu) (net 8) (status 10))
 (segment (start 150.608996 106.68) (end 151.734006 105.55499) (width 0.25) (layer F.Cu) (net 8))
 (segment (start 171.85 96.52) (end 162.2425 96.52) (width 0.25) (layer F.Cu) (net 9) (status 30))
 (segment (start 152.6 96.52) (end 154.618996 96.52) (width 0.25) (layer B.Cu) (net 9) (status 10))
 (segment (start 155.744006 97.64501) (end 157.62499 97.64501) (width 0.25) (layer B.Cu) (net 9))
 (segment (start 154.618996 96.52) (end 155.744006 97.64501) (width 0.25) (layer B.Cu) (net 9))
 (segment (start 158.75 96.52) (end 162.2425 96.52) (width 0.25) (layer B.Cu) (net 9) (status 20))
 (segment (start 157.62499 97.64501) (end 158.75 96.52) (width 0.25) (layer B.Cu) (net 9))
 (segment (start 147.0025 104.14) (end 137.36 104.14) (width 0.25) (layer F.Cu) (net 10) (status 30))
 (segment (start 147.0025 104.14) (end 150.495 104.14) (width 0.25) (layer F.Cu) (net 10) (status 10))
 (segment (start 150.495 104.14) (end 151.13 103.505) (width 0.25) (layer F.Cu) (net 10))
 (segment (start 151.734006 103.01499) (end 153.465994 103.01499) (width 0.25) (layer F.Cu) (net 10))
 (segment (start 151.13 103.505) (end 151.243996 103.505) (width 0.25) (layer F.Cu) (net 10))
 (segment (start 151.243996 103.505) (end 151.734006 103.01499) (width 0.25) (layer F.Cu) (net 10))
 (segment (start 153.465994 103.01499) (end 154.591004 104.14) (width 0.25) (layer F.Cu) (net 10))
 (segment (start 154.591004 104.14) (end 156.61 104.14) (width 0.25) (layer F.Cu) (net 10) (status 20))
 (segment (start 162.2425 99.06) (end 171.85 99.06) (width 0.25) (layer F.Cu) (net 11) (status 30))
 (segment (start 152.6 99.06) (end 154.618996 99.06) (width 0.25) (layer B.Cu) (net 11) (status 10))
 (segment (start 155.744006 100.18501) (end 157.62499 100.18501) (width 0.25) (layer B.Cu) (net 11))
 (segment (start 154.618996 99.06) (end 155.744006 100.18501) (width 0.25) (layer B.Cu) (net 11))
 (segment (start 158.75 99.06) (end 162.2425 99.06) (width 0.25) (layer B.Cu) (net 11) (status 20))
 (segment (start 157.62499 100.18501) (end 158.75 99.06) (width 0.25) (layer B.Cu) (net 11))
 (segment (start 137.36 101.6) (end 147.0025 101.6) (width 0.25) (layer F.Cu) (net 12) (status 30))
 (segment (start 147.0025 101.6) (end 150.495 101.6) (width 0.25) (layer F.Cu) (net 12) (status 10))
 (segment (start 150.495 101.6) (end 151.765 100.33) (width 0.25) (layer F.Cu) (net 12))
 (segment (start 151.765 100.33) (end 153.67 100.33) (width 0.25) (layer F.Cu) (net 12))
 (segment (start 154.94 101.6) (end 156.61 101.6) (width 0.25) (layer F.Cu) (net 12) (status 20))
 (segment (start 153.67 100.33) (end 154.94 101.6) (width 0.25) (layer F.Cu) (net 12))
 (segment (start 171.85 101.6) (end 162.2425 101.6) (width 0.25) (layer F.Cu) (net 13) (status 30))
 (segment (start 157.475994 102.72501) (end 158.601004 101.6) (width 0.25) (layer B.Cu) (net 13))
 (segment (start 155.744006 102.72501) (end 157.475994 102.72501) (width 0.25) (layer B.Cu) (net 13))
 (segment (start 158.601004 101.6) (end 162.2425 101.6) (width 0.25) (layer B.Cu) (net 13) (status 20))
 (segment (start 152.6 101.6) (end 154.618996 101.6) (width 0.25) (layer B.Cu) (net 13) (status 10))
 (segment (start 154.618996 101.6) (end 155.744006 102.72501) (width 0.25) (layer B.Cu) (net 13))
 (segment (start 147.0025 99.06) (end 137.36 99.06) (width 0.25) (layer F.Cu) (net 14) (status 30))
 (segment (start 153.465994 97.93499) (end 154.591004 99.06) (width 0.25) (layer F.Cu) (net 14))
 (segment (start 151.734006 97.93499) (end 153.465994 97.93499) (width 0.25) (layer F.Cu) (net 14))
 (segment (start 154.591004 99.06) (end 156.61 99.06) (width 0.25) (layer F.Cu) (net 14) (status 20))
 (segment (start 147.0025 99.06) (end 150.608996 99.06) (width 0.25) (layer F.Cu) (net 14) (status 10))
 (segment (start 150.608996 99.06) (end 151.734006 97.93499) (width 0.25) (layer F.Cu) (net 14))
 (segment (start 162.2425 104.14) (end 171.85 104.14) (width 0.25) (layer F.Cu) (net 15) (status 30))
 (segment (start 152.6 104.14) (end 154.618996 104.14) (width 0.25) (layer B.Cu) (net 15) (status 10))
 (segment (start 155.744006 105.26501) (end 157.62499 105.26501) (width 0.25) (layer B.Cu) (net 15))
 (segment (start 154.618996 104.14) (end 155.744006 105.26501) (width 0.25) (layer B.Cu) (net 15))
 (segment (start 158.75 104.14) (end 162.2425 104.14) (width 0.25) (layer B.Cu) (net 15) (status 20))
 (segment (start 157.62499 105.26501) (end 158.75 104.14) (width 0.25) (layer B.Cu) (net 15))
 (segment (start 137.36 96.52) (end 147.0025 96.52) (width 0.25) (layer F.Cu) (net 16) (status 30))
 (segment (start 154.591004 96.52) (end 156.61 96.52) (width 0.25) (layer F.Cu) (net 16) (status 20))
 (segment (start 153.465994 95.39499) (end 154.591004 96.52) (width 0.25) (layer F.Cu) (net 16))
 (segment (start 151.734006 95.39499) (end 153.465994 95.39499) (width 0.25) (layer F.Cu) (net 16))
 (segment (start 147.0025 96.52) (end 150.608996 96.52) (width 0.25) (layer F.Cu) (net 16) (status 10))
 (segment (start 150.608996 96.52) (end 151.734006 95.39499) (width 0.25) (layer F.Cu) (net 16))
 (segment (start 171.85 106.68) (end 162.2425 106.68) (width 0.25) (layer F.Cu) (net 17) (status 30))
 (segment (start 158.601004 106.68) (end 162.2425 106.68) (width 0.25) (layer B.Cu) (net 17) (status 20))
 (segment (start 157.475994 107.80501) (end 158.601004 106.68) (width 0.25) (layer B.Cu) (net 17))
 (segment (start 152.6 106.68) (end 154.618996 106.68) (width 0.25) (layer B.Cu) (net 17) (status 10))
 (segment (start 155.744006 107.80501) (end 157.475994 107.80501) (width 0.25) (layer B.Cu) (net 17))
 (segment (start 154.618996 106.68) (end 155.744006 107.80501) (width 0.25) (layer B.Cu) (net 17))
 (segment (start 147.0025 93.98) (end 137.36 93.98) (width 0.25) (layer F.Cu) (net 18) (status 30))
 (segment (start 153.465994 92.85499) (end 154.591004 93.98) (width 0.25) (layer F.Cu) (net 18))
 (segment (start 154.591004 93.98) (end 156.61 93.98) (width 0.25) (layer F.Cu) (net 18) (status 20))
 (segment (start 147.0025 93.98) (end 150.608996 93.98) (width 0.25) (layer F.Cu) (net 18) (status 10))
 (segment (start 151.734006 92.85499) (end 153.465994 92.85499) (width 0.25) (layer F.Cu) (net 18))
 (segment (start 150.608996 93.98) (end 151.734006 92.85499) (width 0.25) (layer F.Cu) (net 18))
 (segment (start 162.2425 109.22) (end 171.85 109.22) (width 0.25) (layer F.Cu) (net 19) (status 30))
 (segment (start 158.601004 109.22) (end 162.2425 109.22) (width 0.25) (layer B.Cu) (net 19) (status 20))
 (segment (start 157.475994 110.34501) (end 158.601004 109.22) (width 0.25) (layer B.Cu) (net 19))
 (segment (start 152.6 109.22) (end 154.618996 109.22) (width 0.25) (layer B.Cu) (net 19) (status 10))
 (segment (start 155.744006 110.34501) (end 157.475994 110.34501) (width 0.25) (layer B.Cu) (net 19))
 (segment (start 154.618996 109.22) (end 155.744006 110.34501) (width 0.25) (layer B.Cu) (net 19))
 (segment (start 137.36 91.44) (end 147.0025 91.44) (width 0.25) (layer F.Cu) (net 20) (status 30))
 (segment (start 154.591004 91.44) (end 156.61 91.44) (width 0.25) (layer F.Cu) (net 20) (status 20))
 (segment (start 151.734006 90.31499) (end 153.465994 90.31499) (width 0.25) (layer F.Cu) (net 20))
 (segment (start 147.0025 91.44) (end 150.608996 91.44) (width 0.25) (layer F.Cu) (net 20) (status 10))
 (segment (start 153.465994 90.31499) (end 154.591004 91.44) (width 0.25) (layer F.Cu) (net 20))
 (segment (start 150.608996 91.44) (end 151.734006 90.31499) (width 0.25) (layer F.Cu) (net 20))
 (segment (start 171.85 111.76) (end 162.2425 111.76) (width 0.25) (layer F.Cu) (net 21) (status 30))
 (segment (start 160.02 111.76) (end 162.2425 111.76) (width 0.25) (layer F.Cu) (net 21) (status 20))
 (segment (start 158.75 110.49) (end 160.02 111.76) (width 0.25) (layer F.Cu) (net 21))
 (segment (start 146.05 110.49) (end 158.75 110.49) (width 0.25) (layer F.Cu) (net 21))
 (segment (start 137.36 109.22) (end 144.78 109.22) (width 0.25) (layer F.Cu) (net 21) (status 10))
 (segment (start 144.78 109.22) (end 146.05 110.49) (width 0.25) (layer F.Cu) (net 21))
 (segment (start 147.0025 88.9) (end 137.36 88.9) (width 0.25) (layer F.Cu) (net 22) (status 30))
 (segment (start 154.591004 88.9) (end 156.61 88.9) (width 0.25) (layer F.Cu) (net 22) (status 20))
 (segment (start 151.734006 87.77499) (end 153.465994 87.77499) (width 0.25) (layer F.Cu) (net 22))
 (segment (start 153.465994 87.77499) (end 154.591004 88.9) (width 0.25) (layer F.Cu) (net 22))
 (segment (start 147.0025 88.9) (end 150.608996 88.9) (width 0.25) (layer F.Cu) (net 22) (status 10))
 (segment (start 150.608996 88.9) (end 151.734006 87.77499) (width 0.25) (layer F.Cu) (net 22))
 (segment (start 162.2425 114.3) (end 171.85 114.3) (width 0.25) (layer F.Cu) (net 23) (status 30))
 (segment (start 158.601004 114.3) (end 162.2425 114.3) (width 0.25) (layer F.Cu) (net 23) (status 20))
 (segment (start 157.475994 115.42501) (end 158.601004 114.3) (width 0.25) (layer F.Cu) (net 23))
 (segment (start 155.744006 115.42501) (end 157.475994 115.42501) (width 0.25) (layer F.Cu) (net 23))
 (segment (start 154.618996 114.3) (end 155.744006 115.42501) (width 0.25) (layer F.Cu) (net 23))
 (segment (start 152.6 114.3) (end 154.618996 114.3) (width 0.25) (layer F.Cu) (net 23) (status 10))
 (segment (start 137.36 86.36) (end 147.0025 86.36) (width 0.75) (layer F.Cu) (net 24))
 (segment (start 154.66 84.81) (end 156.21 86.36) (width 0.75) (layer F.Cu) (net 24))
 (segment (start 150.5025 84.81) (end 154.66 84.81) (width 0.75) (layer F.Cu) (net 24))
 (segment (start 156.21 86.36) (end 156.61 86.36) (width 0.75) (layer F.Cu) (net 24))
 (segment (start 148.9525 86.36) (end 150.5025 84.81) (width 0.75) (layer F.Cu) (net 24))
 (segment (start 147.0025 86.36) (end 148.9525 86.36) (width 0.75) (layer F.Cu) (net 24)))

